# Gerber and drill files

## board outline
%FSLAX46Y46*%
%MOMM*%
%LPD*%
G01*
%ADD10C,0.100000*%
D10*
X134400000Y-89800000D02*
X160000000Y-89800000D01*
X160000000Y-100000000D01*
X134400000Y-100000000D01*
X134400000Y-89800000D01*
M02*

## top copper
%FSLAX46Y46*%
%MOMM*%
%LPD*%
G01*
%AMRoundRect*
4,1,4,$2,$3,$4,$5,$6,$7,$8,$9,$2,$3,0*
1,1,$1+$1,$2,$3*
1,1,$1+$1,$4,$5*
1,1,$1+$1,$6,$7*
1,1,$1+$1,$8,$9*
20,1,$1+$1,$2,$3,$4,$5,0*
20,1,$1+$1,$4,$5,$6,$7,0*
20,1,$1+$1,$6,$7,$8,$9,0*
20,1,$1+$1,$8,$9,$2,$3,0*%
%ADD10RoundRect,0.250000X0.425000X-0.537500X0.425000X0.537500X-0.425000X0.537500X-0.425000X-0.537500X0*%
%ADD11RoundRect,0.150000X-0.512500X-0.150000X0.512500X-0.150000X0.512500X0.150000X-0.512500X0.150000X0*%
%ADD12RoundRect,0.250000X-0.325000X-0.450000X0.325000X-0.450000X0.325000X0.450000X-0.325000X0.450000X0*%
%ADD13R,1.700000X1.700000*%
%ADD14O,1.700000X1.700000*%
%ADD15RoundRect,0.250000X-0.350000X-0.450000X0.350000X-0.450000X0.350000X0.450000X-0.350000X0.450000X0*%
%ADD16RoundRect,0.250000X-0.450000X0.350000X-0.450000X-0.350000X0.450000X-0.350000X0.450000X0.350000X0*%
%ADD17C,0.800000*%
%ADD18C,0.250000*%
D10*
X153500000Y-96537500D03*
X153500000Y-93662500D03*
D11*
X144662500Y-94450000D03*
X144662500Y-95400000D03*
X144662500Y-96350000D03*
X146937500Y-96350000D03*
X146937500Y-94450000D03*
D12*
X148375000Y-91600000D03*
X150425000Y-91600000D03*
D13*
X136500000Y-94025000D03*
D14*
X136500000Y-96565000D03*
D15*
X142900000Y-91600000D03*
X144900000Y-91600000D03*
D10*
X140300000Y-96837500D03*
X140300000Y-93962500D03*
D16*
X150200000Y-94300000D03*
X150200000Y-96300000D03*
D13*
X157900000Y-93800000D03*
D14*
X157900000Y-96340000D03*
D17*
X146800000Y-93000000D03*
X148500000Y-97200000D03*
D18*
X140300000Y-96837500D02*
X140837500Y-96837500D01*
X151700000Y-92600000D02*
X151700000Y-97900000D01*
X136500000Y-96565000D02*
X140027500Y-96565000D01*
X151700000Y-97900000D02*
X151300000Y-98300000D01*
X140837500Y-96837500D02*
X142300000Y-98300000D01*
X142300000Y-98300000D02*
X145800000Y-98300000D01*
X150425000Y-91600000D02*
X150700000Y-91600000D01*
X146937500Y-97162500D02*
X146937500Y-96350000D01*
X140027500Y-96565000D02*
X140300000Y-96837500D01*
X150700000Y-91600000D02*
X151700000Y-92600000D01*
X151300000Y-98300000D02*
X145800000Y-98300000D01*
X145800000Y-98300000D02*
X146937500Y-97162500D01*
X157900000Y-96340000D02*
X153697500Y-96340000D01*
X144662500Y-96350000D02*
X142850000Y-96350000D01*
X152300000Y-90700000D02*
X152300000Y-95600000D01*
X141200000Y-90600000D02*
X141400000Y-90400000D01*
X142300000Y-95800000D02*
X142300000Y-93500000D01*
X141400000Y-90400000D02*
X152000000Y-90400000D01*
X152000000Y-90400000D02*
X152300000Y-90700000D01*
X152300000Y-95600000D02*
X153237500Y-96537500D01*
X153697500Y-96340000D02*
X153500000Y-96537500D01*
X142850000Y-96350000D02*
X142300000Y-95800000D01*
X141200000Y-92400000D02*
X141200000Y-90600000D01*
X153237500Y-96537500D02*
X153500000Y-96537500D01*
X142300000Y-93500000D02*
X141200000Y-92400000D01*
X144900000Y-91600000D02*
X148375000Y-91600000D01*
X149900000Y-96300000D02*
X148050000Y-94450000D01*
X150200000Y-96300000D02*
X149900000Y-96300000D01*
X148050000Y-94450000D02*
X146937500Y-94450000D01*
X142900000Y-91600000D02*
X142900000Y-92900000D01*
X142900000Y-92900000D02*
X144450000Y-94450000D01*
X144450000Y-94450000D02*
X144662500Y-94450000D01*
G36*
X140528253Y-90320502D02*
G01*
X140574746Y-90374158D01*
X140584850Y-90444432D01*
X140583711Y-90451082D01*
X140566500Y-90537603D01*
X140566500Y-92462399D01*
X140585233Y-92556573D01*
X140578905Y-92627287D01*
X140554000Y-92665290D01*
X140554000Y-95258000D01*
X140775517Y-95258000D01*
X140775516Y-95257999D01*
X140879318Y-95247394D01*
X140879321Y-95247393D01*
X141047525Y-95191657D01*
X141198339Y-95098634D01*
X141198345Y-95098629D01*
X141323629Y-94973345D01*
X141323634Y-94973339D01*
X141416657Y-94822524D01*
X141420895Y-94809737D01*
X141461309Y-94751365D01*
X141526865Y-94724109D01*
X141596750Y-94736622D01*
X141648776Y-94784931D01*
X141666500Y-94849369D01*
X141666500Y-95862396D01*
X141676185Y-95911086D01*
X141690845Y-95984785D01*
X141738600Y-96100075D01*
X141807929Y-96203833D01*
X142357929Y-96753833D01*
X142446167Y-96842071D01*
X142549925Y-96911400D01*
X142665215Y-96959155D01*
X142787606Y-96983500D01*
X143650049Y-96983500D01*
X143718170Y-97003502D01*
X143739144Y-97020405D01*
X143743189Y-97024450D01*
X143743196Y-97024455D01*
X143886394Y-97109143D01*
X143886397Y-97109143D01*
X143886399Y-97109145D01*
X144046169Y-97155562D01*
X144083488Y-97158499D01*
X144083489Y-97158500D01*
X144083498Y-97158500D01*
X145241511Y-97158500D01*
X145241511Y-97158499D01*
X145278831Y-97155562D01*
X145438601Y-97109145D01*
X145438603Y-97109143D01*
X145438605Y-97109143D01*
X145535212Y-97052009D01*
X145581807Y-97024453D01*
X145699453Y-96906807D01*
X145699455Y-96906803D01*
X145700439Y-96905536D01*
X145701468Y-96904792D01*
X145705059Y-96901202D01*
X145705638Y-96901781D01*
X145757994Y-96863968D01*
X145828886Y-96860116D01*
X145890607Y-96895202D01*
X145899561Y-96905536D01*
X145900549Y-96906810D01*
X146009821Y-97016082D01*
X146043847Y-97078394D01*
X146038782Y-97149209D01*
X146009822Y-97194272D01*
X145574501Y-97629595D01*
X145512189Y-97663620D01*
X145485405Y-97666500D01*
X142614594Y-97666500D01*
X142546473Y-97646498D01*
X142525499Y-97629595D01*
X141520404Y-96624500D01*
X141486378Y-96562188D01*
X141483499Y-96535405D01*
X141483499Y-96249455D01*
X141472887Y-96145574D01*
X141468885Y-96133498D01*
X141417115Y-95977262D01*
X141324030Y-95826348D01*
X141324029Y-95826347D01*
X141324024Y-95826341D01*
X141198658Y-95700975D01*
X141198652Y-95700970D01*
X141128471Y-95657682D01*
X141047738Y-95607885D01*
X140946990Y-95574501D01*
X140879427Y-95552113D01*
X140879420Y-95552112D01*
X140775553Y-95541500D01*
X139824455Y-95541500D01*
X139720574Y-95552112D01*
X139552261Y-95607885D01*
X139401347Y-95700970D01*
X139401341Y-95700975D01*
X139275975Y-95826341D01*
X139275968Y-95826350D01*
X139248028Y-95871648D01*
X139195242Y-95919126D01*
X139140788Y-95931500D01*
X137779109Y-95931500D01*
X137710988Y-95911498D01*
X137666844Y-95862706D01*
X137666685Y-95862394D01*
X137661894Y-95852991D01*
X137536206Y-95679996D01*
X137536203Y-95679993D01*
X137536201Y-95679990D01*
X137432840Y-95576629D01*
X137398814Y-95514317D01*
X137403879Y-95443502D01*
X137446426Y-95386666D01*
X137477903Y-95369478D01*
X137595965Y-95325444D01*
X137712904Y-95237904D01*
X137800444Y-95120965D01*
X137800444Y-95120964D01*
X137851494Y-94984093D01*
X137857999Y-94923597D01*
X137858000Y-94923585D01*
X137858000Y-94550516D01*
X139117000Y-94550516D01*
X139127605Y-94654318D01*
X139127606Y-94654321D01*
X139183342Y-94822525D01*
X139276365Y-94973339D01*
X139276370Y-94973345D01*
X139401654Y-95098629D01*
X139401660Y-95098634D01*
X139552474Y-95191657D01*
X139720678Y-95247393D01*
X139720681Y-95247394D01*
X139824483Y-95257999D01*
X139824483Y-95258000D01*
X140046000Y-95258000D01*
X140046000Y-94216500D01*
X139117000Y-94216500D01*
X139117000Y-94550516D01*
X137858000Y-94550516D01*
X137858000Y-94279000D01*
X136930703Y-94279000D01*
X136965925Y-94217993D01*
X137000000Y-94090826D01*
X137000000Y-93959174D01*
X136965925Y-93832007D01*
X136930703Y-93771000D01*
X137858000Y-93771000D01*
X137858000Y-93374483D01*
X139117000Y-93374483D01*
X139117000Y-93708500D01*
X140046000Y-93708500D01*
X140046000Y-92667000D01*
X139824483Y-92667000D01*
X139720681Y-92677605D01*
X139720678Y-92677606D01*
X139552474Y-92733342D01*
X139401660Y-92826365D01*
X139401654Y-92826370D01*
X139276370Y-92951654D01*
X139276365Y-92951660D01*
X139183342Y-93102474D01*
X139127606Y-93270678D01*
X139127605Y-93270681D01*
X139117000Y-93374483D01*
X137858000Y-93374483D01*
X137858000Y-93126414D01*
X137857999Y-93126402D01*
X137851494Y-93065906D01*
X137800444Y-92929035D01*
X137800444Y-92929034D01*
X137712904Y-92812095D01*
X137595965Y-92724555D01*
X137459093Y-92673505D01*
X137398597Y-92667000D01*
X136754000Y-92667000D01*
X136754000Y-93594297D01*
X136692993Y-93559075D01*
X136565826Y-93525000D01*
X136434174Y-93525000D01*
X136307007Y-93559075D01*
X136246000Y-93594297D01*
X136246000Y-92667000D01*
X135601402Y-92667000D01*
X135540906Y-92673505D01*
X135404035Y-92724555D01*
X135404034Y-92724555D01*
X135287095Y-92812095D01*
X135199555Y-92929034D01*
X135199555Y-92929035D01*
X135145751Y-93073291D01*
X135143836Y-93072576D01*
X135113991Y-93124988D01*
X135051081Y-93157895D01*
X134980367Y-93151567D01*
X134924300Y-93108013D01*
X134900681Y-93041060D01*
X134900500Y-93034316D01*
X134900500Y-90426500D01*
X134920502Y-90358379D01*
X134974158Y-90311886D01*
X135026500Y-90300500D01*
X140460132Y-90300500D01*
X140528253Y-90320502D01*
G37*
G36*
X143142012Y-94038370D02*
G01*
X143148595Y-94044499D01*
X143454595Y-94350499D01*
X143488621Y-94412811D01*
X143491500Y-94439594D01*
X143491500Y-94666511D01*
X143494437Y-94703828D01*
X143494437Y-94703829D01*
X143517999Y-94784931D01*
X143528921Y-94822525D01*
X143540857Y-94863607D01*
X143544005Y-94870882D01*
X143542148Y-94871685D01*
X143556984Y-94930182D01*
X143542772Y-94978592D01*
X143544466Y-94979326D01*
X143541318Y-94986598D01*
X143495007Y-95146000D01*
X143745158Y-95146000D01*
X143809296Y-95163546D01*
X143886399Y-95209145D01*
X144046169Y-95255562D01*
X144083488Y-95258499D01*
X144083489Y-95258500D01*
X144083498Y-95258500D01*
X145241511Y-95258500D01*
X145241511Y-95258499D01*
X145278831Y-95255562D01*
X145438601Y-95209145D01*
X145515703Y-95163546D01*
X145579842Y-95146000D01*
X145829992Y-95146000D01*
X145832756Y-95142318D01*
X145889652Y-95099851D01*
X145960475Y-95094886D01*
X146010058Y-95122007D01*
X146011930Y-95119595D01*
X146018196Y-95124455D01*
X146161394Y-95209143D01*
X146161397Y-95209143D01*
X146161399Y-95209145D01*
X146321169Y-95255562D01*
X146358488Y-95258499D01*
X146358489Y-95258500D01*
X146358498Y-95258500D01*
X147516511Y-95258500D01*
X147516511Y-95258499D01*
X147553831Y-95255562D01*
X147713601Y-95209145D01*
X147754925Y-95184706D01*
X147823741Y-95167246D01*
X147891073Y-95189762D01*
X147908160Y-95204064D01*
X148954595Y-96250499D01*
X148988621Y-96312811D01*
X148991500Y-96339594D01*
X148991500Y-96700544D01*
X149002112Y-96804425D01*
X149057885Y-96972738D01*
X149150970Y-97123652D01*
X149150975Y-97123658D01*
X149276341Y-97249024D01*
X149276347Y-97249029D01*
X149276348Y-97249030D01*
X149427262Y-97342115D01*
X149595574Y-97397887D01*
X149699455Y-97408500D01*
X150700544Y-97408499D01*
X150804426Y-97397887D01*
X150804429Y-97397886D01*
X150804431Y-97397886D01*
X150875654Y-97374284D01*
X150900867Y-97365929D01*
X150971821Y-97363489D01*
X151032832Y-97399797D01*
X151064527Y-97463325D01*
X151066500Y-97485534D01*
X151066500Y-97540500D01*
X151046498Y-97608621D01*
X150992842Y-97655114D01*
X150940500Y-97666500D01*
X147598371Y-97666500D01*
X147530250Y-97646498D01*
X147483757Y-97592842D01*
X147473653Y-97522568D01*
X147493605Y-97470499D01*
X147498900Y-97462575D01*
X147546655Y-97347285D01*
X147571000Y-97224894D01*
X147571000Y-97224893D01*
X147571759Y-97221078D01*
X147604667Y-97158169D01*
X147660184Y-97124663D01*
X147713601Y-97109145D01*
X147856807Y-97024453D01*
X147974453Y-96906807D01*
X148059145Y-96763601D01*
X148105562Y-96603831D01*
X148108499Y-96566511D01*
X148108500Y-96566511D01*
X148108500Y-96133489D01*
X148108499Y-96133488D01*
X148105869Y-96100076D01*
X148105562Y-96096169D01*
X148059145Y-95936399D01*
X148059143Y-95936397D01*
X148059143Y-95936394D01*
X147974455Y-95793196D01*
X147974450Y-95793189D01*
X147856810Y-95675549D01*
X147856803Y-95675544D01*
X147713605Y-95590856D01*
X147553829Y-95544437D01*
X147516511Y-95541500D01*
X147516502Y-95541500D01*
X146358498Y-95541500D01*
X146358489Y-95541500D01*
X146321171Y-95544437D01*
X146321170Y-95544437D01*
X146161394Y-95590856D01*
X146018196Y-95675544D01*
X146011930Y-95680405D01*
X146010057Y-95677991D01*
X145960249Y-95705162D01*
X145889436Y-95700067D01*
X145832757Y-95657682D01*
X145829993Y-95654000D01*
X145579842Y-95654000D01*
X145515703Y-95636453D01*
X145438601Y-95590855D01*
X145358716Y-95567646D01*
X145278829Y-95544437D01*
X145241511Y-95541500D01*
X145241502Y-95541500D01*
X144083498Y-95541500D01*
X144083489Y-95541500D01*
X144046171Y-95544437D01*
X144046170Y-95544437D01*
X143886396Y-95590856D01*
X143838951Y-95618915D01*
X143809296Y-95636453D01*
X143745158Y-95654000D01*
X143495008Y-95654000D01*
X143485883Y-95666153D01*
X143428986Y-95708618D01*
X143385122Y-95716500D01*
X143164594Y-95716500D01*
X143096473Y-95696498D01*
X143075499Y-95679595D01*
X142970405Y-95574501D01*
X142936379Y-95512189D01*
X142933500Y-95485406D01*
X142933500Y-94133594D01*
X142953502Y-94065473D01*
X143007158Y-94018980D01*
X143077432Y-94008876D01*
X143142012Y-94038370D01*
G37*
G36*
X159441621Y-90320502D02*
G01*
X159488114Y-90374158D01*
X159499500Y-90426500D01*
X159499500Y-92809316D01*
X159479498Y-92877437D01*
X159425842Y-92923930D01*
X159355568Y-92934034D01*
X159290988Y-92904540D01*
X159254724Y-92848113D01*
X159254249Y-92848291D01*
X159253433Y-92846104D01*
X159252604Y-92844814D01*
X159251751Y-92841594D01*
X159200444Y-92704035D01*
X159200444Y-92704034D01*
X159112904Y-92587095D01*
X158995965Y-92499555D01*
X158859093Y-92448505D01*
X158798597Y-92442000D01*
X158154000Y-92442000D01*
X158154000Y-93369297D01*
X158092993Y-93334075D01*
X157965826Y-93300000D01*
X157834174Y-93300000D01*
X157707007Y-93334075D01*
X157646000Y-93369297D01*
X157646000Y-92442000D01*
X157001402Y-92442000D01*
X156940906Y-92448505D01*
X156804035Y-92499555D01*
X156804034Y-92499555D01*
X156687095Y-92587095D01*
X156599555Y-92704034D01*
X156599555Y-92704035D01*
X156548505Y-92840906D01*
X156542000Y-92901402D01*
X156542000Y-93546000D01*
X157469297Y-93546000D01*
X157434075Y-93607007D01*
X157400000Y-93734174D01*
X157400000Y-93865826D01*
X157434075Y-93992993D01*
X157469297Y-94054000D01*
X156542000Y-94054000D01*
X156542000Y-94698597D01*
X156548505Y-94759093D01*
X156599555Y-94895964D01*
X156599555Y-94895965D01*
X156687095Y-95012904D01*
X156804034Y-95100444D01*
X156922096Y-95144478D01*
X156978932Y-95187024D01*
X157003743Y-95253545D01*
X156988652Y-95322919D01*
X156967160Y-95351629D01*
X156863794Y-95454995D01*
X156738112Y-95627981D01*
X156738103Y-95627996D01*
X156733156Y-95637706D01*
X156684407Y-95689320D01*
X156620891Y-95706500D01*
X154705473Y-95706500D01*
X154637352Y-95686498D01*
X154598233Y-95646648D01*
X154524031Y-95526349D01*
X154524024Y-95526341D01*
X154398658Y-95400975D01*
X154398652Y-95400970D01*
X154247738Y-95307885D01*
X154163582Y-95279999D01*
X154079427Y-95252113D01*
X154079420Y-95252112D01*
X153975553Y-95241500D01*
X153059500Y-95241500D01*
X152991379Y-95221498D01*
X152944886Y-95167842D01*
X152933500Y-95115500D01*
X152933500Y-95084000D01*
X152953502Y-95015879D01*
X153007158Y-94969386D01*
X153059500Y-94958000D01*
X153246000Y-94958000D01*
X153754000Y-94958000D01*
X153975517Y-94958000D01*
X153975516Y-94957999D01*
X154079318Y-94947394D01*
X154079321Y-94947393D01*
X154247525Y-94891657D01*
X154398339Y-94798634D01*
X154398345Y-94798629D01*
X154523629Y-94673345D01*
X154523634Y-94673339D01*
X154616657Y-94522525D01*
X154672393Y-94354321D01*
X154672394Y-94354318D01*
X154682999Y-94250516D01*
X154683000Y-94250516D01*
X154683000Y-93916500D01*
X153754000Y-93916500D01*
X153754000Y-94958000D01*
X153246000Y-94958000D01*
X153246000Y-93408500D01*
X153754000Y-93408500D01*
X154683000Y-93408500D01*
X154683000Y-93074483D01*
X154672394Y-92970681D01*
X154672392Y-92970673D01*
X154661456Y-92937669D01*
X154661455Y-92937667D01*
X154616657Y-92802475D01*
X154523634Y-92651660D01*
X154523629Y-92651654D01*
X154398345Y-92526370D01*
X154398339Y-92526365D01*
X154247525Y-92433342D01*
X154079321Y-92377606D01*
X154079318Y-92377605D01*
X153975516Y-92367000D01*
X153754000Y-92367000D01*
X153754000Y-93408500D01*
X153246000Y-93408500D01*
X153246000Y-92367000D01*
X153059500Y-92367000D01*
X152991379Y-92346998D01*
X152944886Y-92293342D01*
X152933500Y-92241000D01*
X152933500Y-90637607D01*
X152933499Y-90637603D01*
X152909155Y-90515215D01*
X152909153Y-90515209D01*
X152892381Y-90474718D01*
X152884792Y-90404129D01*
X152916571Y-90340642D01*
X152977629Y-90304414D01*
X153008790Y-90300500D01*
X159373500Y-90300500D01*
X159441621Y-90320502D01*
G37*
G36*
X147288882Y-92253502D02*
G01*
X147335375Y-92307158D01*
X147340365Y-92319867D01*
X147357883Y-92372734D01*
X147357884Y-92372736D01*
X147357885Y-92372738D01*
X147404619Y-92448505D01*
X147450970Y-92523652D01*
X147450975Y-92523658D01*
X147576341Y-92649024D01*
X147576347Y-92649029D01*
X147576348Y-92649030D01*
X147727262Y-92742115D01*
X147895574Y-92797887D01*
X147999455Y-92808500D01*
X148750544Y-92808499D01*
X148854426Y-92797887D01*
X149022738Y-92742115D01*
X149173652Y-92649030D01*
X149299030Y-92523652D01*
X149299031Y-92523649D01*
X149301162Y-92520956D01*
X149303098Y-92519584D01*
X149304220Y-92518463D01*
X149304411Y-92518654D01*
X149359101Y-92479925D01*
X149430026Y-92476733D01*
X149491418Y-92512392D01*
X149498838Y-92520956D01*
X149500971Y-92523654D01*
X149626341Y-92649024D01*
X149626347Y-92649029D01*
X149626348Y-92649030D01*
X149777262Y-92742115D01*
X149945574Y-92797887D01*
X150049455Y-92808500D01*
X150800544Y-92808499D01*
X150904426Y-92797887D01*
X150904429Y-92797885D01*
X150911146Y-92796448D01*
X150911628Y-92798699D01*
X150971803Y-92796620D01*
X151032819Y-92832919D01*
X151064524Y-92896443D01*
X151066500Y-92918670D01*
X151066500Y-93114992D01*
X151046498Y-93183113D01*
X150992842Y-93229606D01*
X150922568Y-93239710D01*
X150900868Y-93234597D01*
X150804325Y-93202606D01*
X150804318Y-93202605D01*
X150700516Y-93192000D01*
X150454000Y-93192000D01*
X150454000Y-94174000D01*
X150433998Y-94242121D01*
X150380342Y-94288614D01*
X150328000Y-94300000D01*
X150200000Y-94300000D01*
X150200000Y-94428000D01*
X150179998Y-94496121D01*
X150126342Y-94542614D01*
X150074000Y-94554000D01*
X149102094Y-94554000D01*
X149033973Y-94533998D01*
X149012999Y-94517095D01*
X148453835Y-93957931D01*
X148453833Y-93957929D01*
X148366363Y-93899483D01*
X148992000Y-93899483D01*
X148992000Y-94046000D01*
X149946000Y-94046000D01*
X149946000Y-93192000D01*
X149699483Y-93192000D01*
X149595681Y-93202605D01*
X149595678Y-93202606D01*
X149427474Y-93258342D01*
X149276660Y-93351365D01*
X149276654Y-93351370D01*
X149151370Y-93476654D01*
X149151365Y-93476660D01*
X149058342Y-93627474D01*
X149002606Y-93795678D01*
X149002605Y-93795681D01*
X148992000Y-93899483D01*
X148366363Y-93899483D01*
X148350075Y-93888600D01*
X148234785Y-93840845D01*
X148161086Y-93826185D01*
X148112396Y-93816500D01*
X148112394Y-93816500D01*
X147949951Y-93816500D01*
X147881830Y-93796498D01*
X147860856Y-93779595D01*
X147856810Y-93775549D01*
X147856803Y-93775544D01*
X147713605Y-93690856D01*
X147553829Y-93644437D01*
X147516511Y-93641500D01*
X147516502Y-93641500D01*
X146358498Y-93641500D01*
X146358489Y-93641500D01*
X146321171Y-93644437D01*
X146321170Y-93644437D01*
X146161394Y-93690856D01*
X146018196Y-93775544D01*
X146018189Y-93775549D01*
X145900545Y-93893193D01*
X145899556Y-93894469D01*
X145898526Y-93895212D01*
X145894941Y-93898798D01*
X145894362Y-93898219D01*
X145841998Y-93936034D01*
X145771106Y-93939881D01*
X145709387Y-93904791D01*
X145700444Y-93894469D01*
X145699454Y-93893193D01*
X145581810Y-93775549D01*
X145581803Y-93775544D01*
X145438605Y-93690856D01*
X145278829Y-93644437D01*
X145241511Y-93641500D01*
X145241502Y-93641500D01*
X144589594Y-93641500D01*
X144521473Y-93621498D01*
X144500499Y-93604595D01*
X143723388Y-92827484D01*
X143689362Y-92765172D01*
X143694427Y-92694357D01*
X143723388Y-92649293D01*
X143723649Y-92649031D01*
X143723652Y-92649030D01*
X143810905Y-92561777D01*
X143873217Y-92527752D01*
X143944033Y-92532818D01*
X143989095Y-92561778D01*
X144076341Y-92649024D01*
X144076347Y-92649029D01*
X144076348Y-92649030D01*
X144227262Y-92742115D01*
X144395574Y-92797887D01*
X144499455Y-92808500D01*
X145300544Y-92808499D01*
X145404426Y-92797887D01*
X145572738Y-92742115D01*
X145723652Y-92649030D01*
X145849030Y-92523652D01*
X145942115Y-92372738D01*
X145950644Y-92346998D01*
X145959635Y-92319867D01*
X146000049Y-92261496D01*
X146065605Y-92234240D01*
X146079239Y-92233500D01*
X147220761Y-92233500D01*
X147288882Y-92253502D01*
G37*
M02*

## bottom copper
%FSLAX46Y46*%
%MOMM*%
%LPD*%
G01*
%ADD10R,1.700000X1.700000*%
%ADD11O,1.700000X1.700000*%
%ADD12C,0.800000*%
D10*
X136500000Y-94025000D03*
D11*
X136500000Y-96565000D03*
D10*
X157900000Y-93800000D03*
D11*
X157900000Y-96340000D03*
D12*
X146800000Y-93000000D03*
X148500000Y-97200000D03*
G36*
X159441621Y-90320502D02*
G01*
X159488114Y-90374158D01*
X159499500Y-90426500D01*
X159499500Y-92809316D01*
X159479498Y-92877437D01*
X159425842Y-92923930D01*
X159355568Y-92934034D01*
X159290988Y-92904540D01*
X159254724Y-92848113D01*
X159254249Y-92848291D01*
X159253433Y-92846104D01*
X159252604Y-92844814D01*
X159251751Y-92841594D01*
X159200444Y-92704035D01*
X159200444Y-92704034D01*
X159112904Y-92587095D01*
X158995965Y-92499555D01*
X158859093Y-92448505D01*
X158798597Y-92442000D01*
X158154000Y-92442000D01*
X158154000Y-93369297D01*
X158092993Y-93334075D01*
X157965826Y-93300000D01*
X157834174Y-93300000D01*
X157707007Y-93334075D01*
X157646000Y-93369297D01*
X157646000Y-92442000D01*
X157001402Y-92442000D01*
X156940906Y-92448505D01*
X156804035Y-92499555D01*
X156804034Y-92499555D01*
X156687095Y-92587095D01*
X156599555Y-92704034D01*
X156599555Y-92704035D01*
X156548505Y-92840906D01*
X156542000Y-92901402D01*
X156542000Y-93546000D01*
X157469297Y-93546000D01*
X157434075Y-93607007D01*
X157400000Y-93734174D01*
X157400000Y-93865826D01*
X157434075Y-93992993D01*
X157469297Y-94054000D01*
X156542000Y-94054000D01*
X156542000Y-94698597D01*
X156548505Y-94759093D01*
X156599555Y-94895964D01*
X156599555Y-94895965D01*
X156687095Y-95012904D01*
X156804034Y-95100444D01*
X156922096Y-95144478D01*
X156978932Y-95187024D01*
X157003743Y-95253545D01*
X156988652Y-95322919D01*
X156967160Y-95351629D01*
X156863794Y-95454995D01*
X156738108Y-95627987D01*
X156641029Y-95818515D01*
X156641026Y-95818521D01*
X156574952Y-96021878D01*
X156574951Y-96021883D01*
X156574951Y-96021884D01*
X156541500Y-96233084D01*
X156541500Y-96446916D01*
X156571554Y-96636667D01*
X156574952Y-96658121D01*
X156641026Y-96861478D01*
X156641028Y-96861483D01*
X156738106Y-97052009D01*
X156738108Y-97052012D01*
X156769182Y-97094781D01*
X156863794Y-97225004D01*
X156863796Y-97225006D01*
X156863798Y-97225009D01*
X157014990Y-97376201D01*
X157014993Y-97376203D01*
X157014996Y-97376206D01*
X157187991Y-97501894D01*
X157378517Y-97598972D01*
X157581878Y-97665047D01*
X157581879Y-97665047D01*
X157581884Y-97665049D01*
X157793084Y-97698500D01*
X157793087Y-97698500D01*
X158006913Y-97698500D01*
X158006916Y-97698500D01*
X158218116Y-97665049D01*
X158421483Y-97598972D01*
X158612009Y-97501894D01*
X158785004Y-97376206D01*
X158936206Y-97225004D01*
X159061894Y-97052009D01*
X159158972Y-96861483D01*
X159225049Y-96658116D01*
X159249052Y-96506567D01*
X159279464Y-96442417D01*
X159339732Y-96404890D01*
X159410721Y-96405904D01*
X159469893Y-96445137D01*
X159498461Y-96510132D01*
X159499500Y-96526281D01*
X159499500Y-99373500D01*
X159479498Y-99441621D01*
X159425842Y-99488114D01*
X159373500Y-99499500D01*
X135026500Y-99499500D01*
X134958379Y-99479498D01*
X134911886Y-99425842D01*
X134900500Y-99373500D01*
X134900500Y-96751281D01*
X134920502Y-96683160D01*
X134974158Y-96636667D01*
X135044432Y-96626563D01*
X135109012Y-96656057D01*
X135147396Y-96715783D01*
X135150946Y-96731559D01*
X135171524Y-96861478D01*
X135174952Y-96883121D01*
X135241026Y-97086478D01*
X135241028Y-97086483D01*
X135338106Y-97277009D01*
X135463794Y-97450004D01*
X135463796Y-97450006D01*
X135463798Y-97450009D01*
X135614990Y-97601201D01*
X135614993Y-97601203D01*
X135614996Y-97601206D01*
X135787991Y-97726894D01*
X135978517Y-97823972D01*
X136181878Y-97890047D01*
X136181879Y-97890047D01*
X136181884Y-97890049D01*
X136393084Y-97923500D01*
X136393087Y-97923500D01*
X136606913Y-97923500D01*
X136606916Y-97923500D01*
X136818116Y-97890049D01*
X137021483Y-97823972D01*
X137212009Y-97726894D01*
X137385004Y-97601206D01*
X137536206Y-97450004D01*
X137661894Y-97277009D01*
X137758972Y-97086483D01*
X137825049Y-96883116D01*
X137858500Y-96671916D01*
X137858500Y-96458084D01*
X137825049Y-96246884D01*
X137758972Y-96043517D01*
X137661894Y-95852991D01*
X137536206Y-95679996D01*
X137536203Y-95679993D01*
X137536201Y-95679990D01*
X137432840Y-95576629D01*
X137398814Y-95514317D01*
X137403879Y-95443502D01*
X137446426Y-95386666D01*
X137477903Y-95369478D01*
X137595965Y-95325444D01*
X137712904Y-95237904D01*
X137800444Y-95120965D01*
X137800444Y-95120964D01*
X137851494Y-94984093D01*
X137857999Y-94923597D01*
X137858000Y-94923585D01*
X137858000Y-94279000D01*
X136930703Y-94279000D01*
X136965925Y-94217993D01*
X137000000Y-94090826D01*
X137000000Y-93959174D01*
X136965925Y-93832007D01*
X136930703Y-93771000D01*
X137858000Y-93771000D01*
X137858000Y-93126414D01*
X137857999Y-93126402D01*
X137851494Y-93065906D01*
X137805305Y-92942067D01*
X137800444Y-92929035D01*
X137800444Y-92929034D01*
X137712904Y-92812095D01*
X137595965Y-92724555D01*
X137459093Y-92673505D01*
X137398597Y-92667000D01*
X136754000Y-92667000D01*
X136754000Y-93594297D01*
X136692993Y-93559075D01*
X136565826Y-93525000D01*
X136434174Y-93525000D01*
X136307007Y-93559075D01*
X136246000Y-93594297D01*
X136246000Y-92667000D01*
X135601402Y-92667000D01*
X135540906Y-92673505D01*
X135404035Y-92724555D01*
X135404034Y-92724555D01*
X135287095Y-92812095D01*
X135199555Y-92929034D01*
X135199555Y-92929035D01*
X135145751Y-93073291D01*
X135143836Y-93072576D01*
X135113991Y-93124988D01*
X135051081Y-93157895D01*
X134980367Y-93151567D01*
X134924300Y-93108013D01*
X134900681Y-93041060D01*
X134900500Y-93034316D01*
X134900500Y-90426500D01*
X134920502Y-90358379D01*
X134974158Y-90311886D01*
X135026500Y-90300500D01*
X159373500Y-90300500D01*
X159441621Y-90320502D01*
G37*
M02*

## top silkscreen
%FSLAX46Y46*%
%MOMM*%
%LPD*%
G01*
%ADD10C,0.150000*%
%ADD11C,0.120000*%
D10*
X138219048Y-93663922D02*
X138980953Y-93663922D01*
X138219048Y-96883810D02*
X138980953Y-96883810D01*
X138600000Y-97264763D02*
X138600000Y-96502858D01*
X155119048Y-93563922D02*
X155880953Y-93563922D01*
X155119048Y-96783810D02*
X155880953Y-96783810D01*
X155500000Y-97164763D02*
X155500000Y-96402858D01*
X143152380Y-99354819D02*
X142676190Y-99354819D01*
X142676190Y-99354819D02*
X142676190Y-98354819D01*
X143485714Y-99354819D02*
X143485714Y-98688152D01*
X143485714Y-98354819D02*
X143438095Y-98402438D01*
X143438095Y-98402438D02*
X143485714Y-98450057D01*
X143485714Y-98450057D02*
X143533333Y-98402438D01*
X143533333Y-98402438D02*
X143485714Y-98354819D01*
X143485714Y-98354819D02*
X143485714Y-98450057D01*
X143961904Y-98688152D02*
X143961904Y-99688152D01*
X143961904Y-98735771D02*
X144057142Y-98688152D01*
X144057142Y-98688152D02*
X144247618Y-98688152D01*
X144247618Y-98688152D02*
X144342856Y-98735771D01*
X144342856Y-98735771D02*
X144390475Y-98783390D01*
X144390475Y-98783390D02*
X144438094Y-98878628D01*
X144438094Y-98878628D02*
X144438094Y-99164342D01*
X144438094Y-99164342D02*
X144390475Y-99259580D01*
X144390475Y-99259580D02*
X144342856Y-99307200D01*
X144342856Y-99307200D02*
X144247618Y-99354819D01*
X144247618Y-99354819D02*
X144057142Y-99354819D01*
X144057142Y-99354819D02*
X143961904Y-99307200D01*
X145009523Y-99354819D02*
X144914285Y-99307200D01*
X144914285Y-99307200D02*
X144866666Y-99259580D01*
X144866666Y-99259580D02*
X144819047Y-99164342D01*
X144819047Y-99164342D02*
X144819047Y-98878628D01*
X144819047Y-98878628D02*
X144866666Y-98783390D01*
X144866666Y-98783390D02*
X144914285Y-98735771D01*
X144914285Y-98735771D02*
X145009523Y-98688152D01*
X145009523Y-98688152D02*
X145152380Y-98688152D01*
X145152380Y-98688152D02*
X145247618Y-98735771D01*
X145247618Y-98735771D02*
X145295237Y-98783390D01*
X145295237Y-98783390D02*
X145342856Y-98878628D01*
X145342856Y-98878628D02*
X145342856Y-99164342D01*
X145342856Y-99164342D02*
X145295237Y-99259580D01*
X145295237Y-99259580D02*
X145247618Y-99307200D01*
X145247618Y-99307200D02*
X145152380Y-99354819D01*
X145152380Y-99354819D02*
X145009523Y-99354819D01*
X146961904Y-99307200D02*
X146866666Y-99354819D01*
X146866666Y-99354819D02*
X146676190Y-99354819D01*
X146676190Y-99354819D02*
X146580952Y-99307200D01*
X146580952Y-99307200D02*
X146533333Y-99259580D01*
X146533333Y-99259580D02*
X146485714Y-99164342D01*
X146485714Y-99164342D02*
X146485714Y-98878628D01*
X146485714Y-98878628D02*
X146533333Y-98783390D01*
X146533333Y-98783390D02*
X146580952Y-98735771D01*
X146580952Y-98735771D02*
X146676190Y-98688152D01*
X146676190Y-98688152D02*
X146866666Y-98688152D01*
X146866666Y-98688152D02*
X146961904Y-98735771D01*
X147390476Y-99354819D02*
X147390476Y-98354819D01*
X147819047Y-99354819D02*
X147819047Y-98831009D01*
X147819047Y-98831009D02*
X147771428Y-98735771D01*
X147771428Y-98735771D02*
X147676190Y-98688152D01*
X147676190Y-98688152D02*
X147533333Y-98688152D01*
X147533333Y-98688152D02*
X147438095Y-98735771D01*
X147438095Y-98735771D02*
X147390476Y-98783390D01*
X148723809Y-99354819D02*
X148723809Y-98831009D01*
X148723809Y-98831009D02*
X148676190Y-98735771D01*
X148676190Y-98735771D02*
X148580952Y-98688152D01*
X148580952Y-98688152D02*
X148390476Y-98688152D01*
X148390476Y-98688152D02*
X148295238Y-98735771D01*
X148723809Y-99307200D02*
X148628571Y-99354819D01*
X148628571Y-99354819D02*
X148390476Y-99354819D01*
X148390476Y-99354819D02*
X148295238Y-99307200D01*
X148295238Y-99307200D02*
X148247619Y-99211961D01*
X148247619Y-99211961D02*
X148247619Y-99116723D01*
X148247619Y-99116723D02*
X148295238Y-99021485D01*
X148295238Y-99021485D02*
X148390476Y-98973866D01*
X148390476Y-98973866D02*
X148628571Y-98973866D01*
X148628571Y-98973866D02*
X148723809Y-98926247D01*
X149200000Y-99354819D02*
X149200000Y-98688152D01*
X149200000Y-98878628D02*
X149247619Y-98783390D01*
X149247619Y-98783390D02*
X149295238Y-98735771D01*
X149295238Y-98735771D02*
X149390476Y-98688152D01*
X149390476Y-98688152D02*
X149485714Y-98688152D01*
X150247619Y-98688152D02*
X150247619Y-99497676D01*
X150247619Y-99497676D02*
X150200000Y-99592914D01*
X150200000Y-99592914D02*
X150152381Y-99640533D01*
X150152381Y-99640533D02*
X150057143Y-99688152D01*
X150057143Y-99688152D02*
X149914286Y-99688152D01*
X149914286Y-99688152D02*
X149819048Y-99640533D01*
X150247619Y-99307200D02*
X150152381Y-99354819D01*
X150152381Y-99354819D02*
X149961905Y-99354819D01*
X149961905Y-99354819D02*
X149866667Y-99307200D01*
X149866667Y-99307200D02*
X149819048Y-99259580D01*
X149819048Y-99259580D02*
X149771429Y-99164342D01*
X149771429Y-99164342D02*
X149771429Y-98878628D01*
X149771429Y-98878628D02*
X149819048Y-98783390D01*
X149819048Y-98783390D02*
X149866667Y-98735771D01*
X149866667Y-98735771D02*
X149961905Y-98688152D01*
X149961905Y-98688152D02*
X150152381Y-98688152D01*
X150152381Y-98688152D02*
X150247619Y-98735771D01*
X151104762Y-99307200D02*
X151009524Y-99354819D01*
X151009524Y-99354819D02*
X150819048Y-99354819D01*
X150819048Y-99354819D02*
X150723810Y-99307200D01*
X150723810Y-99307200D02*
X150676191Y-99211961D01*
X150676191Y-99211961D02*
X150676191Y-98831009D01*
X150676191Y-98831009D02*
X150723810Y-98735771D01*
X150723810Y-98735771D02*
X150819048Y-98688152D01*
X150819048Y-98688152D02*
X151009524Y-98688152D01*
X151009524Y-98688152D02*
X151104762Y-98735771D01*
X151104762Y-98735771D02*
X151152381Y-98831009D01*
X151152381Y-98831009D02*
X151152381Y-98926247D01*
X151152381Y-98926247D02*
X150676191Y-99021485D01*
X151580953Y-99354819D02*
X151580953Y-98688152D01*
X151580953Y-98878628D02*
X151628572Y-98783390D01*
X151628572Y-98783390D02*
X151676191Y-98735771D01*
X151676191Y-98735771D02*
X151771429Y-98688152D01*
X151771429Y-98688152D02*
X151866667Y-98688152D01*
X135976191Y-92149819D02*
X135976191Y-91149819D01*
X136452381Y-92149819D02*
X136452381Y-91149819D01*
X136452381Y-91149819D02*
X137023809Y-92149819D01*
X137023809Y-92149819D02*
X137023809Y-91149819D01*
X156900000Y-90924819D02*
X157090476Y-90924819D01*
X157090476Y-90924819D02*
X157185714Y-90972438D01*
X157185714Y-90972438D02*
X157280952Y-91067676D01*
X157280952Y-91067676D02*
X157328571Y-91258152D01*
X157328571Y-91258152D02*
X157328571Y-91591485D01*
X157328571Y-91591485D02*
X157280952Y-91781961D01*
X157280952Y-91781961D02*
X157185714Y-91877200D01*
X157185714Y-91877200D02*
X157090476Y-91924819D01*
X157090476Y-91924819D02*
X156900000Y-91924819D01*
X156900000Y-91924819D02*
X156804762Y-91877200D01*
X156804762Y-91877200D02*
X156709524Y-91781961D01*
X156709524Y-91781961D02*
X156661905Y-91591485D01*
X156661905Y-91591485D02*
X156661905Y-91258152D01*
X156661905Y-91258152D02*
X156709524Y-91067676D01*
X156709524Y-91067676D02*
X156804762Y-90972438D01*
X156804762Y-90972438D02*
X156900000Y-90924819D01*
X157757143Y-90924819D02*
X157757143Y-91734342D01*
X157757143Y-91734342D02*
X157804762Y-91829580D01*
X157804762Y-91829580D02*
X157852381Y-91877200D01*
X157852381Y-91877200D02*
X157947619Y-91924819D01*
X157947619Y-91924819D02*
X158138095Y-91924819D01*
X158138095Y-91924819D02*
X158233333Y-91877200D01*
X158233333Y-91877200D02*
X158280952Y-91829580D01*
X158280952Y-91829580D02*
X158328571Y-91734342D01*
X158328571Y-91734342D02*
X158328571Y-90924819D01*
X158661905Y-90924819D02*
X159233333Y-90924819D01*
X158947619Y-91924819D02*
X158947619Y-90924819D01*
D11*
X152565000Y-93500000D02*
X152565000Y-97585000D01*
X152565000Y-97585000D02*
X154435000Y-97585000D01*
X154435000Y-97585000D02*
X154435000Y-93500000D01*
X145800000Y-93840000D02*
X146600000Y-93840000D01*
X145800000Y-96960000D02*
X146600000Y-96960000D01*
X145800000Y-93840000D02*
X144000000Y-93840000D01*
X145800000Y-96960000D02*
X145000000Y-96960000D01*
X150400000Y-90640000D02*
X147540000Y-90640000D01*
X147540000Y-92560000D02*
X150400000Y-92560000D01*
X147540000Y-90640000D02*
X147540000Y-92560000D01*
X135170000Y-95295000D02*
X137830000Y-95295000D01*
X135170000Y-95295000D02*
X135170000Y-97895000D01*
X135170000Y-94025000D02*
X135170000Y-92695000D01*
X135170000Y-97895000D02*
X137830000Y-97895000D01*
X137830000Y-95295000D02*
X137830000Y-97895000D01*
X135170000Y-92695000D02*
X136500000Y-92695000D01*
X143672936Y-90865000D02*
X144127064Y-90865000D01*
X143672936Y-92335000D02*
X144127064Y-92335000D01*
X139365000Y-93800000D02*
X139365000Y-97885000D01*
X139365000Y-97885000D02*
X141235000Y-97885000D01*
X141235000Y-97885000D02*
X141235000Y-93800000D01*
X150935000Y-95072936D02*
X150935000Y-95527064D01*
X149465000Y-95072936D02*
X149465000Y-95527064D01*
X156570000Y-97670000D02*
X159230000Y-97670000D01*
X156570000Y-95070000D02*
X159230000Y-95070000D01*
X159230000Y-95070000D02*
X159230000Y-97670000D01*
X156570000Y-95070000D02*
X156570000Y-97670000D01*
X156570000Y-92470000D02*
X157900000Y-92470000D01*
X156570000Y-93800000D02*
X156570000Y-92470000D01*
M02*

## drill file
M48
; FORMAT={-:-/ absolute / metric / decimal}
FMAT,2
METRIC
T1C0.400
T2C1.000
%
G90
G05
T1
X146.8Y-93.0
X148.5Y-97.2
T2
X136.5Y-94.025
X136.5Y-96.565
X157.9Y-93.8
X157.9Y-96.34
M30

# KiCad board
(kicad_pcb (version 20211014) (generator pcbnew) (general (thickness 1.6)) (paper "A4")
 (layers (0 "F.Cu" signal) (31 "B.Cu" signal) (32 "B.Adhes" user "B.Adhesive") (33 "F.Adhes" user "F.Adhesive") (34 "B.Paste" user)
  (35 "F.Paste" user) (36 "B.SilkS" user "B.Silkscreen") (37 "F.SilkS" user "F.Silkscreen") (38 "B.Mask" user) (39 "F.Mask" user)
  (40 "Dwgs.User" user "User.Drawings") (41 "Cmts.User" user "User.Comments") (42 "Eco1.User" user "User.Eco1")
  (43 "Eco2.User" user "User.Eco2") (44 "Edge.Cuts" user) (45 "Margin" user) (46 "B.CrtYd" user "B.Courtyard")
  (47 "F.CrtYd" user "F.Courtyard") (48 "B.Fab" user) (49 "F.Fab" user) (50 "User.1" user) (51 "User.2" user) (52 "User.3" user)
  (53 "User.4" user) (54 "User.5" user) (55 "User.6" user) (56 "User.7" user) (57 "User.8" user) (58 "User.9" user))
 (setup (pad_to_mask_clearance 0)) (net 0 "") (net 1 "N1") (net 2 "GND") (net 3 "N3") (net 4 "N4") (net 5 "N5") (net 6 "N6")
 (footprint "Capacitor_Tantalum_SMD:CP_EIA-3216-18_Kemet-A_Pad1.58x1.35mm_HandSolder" (layer "F.Cu") (at 153.5 95.1 90)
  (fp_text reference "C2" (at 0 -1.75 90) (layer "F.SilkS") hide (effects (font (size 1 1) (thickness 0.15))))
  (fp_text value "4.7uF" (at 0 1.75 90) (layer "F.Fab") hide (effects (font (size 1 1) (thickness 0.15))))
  (fp_line (start 1.6 -0.935) (end -2.485 -0.935) (layer "F.SilkS") (width 0.12))
  (fp_line (start -2.485 -0.935) (end -2.485 0.935) (layer "F.SilkS") (width 0.12))
  (fp_line (start -2.485 0.935) (end 1.6 0.935) (layer "F.SilkS") (width 0.12))
  (pad "1" smd roundrect (at -1.4375 0 90) (size 1.575 1.35) (layers "F.Cu" "F.Paste" "F.Mask") (roundrect_rratio 0.1851851852) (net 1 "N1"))
  (pad "2" smd roundrect (at 1.4375 0 90) (size 1.575 1.35) (layers "F.Cu" "F.Paste" "F.Mask") (roundrect_rratio 0.1851851852) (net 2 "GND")))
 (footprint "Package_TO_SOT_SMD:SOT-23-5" (layer "F.Cu") (at 145.8 95.4)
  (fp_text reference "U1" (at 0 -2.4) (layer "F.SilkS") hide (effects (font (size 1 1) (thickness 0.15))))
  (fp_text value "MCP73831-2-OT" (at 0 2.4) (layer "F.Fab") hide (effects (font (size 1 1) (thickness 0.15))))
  (fp_line (start 0 -1.56) (end 0.8 -1.56) (layer "F.SilkS") (width 0.12))
  (fp_line (start 0 1.56) (end 0.8 1.56) (layer "F.SilkS") (width 0.12))
  (fp_line (start 0 -1.56) (end -1.8 -1.56) (layer "F.SilkS") (width 0.12))
  (fp_line (start 0 1.56) (end -0.8 1.56) (layer "F.SilkS") (width 0.12))
  (pad "1" smd roundrect (at -1.1375 -0.95) (size 1.325 0.6) (layers "F.Cu" "F.Paste" "F.Mask") (roundrect_rratio 0.25) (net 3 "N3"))
  (pad "2" smd roundrect (at -1.1375 0) (size 1.325 0.6) (layers "F.Cu" "F.Paste" "F.Mask") (roundrect_rratio 0.25) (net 2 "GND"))
  (pad "3" smd roundrect (at -1.1375 0.95) (size 1.325 0.6) (layers "F.Cu" "F.Paste" "F.Mask") (roundrect_rratio 0.25) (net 1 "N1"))
  (pad "4" smd roundrect (at 1.1375 0.95) (size 1.325 0.6) (layers "F.Cu" "F.Paste" "F.Mask") (roundrect_rratio 0.25) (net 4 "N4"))
  (pad "5" smd roundrect (at 1.1375 -0.95) (size 1.325 0.6) (layers "F.Cu" "F.Paste" "F.Mask") (roundrect_rratio 0.25) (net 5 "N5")))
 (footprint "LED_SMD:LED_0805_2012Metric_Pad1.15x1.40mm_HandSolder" (layer "F.Cu") (at 149.4 91.6)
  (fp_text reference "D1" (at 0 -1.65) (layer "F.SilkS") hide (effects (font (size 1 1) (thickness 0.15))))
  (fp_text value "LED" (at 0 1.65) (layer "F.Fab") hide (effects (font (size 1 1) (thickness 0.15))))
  (fp_line (start 1 -0.96) (end -1.86 -0.96) (layer "F.SilkS") (width 0.12))
  (fp_line (start -1.86 0.96) (end 1 0.96) (layer "F.SilkS") (width 0.12))
  (fp_line (start -1.86 -0.96) (end -1.86 0.96) (layer "F.SilkS") (width 0.12))
  (pad "1" smd roundrect (at -1.025 0) (size 1.15 1.4) (layers "F.Cu" "F.Paste" "F.Mask") (roundrect_rratio 0.2173913043) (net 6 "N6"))
  (pad "2" smd roundrect (at 1.025 0) (size 1.15 1.4) (layers "F.Cu" "F.Paste" "F.Mask") (roundrect_rratio 0.2173913043) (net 4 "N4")))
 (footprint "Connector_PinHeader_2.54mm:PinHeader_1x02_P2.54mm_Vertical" (layer "F.Cu") (at 136.5 94.025)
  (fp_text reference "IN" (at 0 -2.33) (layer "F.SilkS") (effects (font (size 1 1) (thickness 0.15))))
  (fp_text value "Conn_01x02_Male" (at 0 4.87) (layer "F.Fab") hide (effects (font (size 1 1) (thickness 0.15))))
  (fp_line (start -1.33 1.27) (end 1.33 1.27) (layer "F.SilkS") (width 0.12))
  (fp_line (start -1.33 1.27) (end -1.33 3.87) (layer "F.SilkS") (width 0.12))
  (fp_line (start -1.33 0) (end -1.33 -1.33) (layer "F.SilkS") (width 0.12))
  (fp_line (start -1.33 3.87) (end 1.33 3.87) (layer "F.SilkS") (width 0.12))
  (fp_line (start 1.33 1.27) (end 1.33 3.87) (layer "F.SilkS") (width 0.12))
  (fp_line (start -1.33 -1.33) (end 0 -1.33) (layer "F.SilkS") (width 0.12))
  (pad "1" thru_hole rect (at 0 0) (size 1.7 1.7) (drill 1) (layers *.Cu *.Mask) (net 2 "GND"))
  (pad "2" thru_hole oval (at 0 2.54) (size 1.7 1.7) (drill 1) (layers *.Cu *.Mask) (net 4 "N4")))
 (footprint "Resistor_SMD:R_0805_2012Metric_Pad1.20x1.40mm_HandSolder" (layer "F.Cu") (at 143.9 91.6)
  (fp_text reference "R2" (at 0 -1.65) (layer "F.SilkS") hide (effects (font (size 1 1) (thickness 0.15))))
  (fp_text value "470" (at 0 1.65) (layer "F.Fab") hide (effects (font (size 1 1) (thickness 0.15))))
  (fp_line (start -0.227064 -0.735) (end 0.227064 -0.735) (layer "F.SilkS") (width 0.12))
  (fp_line (start -0.227064 0.735) (end 0.227064 0.735) (layer "F.SilkS") (width 0.12))
  (pad "1" smd roundrect (at -1 0) (size 1.2 1.4) (layers "F.Cu" "F.Paste" "F.Mask") (roundrect_rratio 0.2083333333) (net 3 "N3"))
  (pad "2" smd roundrect (at 1 0) (size 1.2 1.4) (layers "F.Cu" "F.Paste" "F.Mask") (roundrect_rratio 0.2083333333) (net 6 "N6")))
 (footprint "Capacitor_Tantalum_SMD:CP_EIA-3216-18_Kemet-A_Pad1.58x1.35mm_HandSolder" (layer "F.Cu") (at 140.3 95.4 90)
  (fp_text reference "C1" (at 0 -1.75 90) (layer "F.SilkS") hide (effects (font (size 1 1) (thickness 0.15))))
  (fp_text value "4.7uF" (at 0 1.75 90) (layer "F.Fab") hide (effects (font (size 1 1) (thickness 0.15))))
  (fp_line (start 1.6 -0.935) (end -2.485 -0.935) (layer "F.SilkS") (width 0.12))
  (fp_line (start -2.485 -0.935) (end -2.485 0.935) (layer "F.SilkS") (width 0.12))
  (fp_line (start -2.485 0.935) (end 1.6 0.935) (layer "F.SilkS") (width 0.12))
  (pad "1" smd roundrect (at -1.4375 0 90) (size 1.575 1.35) (layers "F.Cu" "F.Paste" "F.Mask") (roundrect_rratio 0.1851851852) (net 4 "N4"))
  (pad "2" smd roundrect (at 1.4375 0 90) (size 1.575 1.35) (layers "F.Cu" "F.Paste" "F.Mask") (roundrect_rratio 0.1851851852) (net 2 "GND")))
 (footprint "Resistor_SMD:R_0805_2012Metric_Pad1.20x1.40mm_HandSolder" (layer "F.Cu") (at 150.2 95.3 -90)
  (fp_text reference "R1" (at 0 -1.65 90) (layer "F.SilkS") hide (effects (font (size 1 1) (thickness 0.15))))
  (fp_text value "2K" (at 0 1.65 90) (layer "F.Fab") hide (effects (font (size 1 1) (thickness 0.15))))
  (fp_line (start -0.227064 -0.735) (end 0.227064 -0.735) (layer "F.SilkS") (width 0.12))
  (fp_line (start -0.227064 0.735) (end 0.227064 0.735) (layer "F.SilkS") (width 0.12))
  (pad "1" smd roundrect (at -1 0 270) (size 1.2 1.4) (layers "F.Cu" "F.Paste" "F.Mask") (roundrect_rratio 0.2083333333) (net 2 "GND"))
  (pad "2" smd roundrect (at 1 0 270) (size 1.2 1.4) (layers "F.Cu" "F.Paste" "F.Mask") (roundrect_rratio 0.2083333333) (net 5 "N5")))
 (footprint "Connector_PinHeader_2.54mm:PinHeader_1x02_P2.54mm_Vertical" (layer "F.Cu") (at 157.9 93.8)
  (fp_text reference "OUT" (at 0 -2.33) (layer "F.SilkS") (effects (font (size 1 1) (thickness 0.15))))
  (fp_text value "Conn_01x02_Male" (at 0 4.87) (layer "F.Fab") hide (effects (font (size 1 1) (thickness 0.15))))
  (fp_line (start -1.33 3.87) (end 1.33 3.87) (layer "F.SilkS") (width 0.12))
  (fp_line (start -1.33 1.27) (end 1.33 1.27) (layer "F.SilkS") (width 0.12))
  (fp_line (start 1.33 1.27) (end 1.33 3.87) (layer "F.SilkS") (width 0.12))
  (fp_line (start -1.33 1.27) (end -1.33 3.87) (layer "F.SilkS") (width 0.12))
  (fp_line (start -1.33 -1.33) (end 0 -1.33) (layer "F.SilkS") (width 0.12))
  (fp_line (start -1.33 0) (end -1.33 -1.33) (layer "F.SilkS") (width 0.12))
  (pad "1" thru_hole rect (at 0 0) (size 1.7 1.7) (drill 1) (layers *.Cu *.Mask) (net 2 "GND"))
  (pad "2" thru_hole oval (at 0 2.54) (size 1.7 1.7) (drill 1) (layers *.Cu *.Mask) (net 1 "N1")))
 (gr_rect (start 134.4 89.8) (end 160 100) (layer "Edge.Cuts") (width 0.1) (fill none))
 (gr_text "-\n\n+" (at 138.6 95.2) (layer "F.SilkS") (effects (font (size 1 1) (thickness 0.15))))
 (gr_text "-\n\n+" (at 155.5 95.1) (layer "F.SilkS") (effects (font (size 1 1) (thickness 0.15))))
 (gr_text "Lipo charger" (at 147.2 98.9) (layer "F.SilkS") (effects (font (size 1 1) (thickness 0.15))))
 (segment (start 140.3 96.8375) (end 140.8375 96.8375) (width 0.25) (layer "F.Cu") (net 4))
 (segment (start 151.7 92.6) (end 151.7 97.9) (width 0.25) (layer "F.Cu") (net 4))
 (segment (start 136.5 96.565) (end 140.0275 96.565) (width 0.25) (layer "F.Cu") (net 4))
 (segment (start 151.7 97.9) (end 151.3 98.3) (width 0.25) (layer "F.Cu") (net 4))
 (segment (start 140.8375 96.8375) (end 142.3 98.3) (width 0.25) (layer "F.Cu") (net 4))
 (segment (start 142.3 98.3) (end 145.8 98.3) (width 0.25) (layer "F.Cu") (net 4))
 (segment (start 150.425 91.6) (end 150.7 91.6) (width 0.25) (layer "F.Cu") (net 4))
 (segment (start 146.9375 97.1625) (end 146.9375 96.35) (width 0.25) (layer "F.Cu") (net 4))
 (segment (start 140.0275 96.565) (end 140.3 96.8375) (width 0.25) (layer "F.Cu") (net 4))
 (segment (start 150.7 91.6) (end 151.7 92.6) (width 0.25) (layer "F.Cu") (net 4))
 (segment (start 151.3 98.3) (end 145.8 98.3) (width 0.25) (layer "F.Cu") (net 4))
 (segment (start 145.8 98.3) (end 146.9375 97.1625) (width 0.25) (layer "F.Cu") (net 4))
 (via (at 146.8 93) (size 0.8) (drill 0.4) (layers "F.Cu" "B.Cu") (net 2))
 (via (at 148.5 97.2) (size 0.8) (drill 0.4) (layers "F.Cu" "B.Cu") (free) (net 2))
 (segment (start 157.9 96.34) (end 153.6975 96.34) (width 0.25) (layer "F.Cu") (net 1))
 (segment (start 144.6625 96.35) (end 142.85 96.35) (width 0.25) (layer "F.Cu") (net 1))
 (segment (start 152.3 90.7) (end 152.3 95.6) (width 0.25) (layer "F.Cu") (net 1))
 (segment (start 141.2 90.6) (end 141.4 90.4) (width 0.25) (layer "F.Cu") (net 1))
 (segment (start 142.3 95.8) (end 142.3 93.5) (width 0.25) (layer "F.Cu") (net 1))
 (segment (start 141.4 90.4) (end 152 90.4) (width 0.25) (layer "F.Cu") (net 1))
 (segment (start 152 90.4) (end 152.3 90.7) (width 0.25) (layer "F.Cu") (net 1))
 (segment (start 152.3 95.6) (end 153.2375 96.5375) (width 0.25) (layer "F.Cu") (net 1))
 (segment (start 153.6975 96.34) (end 153.5 96.5375) (width 0.25) (layer "F.Cu") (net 1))
 (segment (start 142.85 96.35) (end 142.3 95.8) (width 0.25) (layer "F.Cu") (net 1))
 (segment (start 141.2 92.4) (end 141.2 90.6) (width 0.25) (layer "F.Cu") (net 1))
 (segment (start 153.2375 96.5375) (end 153.5 96.5375) (width 0.25) (layer "F.Cu") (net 1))
 (segment (start 142.3 93.5) (end 141.2 92.4) (width 0.25) (layer "F.Cu") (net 1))
 (segment (start 144.9 91.6) (end 148.375 91.6) (width 0.25) (layer "F.Cu") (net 6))
 (segment (start 149.9 96.3) (end 148.05 94.45) (width 0.25) (layer "F.Cu") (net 5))
 (segment (start 150.2 96.3) (end 149.9 96.3) (width 0.25) (layer "F.Cu") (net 5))
 (segment (start 148.05 94.45) (end 146.9375 94.45) (width 0.25) (layer "F.Cu") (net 5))
 (segment (start 142.9 91.6) (end 142.9 92.9) (width 0.25) (layer "F.Cu") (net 3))
 (segment (start 142.9 92.9) (end 144.45 94.45) (width 0.25) (layer "F.Cu") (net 3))
 (segment (start 144.45 94.45) (end 144.6625 94.45) (width 0.25) (layer "F.Cu") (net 3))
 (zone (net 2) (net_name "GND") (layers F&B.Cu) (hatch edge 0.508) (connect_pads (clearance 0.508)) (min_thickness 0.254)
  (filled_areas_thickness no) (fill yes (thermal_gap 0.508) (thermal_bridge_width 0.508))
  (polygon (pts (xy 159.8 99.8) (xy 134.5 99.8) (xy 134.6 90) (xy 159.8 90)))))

